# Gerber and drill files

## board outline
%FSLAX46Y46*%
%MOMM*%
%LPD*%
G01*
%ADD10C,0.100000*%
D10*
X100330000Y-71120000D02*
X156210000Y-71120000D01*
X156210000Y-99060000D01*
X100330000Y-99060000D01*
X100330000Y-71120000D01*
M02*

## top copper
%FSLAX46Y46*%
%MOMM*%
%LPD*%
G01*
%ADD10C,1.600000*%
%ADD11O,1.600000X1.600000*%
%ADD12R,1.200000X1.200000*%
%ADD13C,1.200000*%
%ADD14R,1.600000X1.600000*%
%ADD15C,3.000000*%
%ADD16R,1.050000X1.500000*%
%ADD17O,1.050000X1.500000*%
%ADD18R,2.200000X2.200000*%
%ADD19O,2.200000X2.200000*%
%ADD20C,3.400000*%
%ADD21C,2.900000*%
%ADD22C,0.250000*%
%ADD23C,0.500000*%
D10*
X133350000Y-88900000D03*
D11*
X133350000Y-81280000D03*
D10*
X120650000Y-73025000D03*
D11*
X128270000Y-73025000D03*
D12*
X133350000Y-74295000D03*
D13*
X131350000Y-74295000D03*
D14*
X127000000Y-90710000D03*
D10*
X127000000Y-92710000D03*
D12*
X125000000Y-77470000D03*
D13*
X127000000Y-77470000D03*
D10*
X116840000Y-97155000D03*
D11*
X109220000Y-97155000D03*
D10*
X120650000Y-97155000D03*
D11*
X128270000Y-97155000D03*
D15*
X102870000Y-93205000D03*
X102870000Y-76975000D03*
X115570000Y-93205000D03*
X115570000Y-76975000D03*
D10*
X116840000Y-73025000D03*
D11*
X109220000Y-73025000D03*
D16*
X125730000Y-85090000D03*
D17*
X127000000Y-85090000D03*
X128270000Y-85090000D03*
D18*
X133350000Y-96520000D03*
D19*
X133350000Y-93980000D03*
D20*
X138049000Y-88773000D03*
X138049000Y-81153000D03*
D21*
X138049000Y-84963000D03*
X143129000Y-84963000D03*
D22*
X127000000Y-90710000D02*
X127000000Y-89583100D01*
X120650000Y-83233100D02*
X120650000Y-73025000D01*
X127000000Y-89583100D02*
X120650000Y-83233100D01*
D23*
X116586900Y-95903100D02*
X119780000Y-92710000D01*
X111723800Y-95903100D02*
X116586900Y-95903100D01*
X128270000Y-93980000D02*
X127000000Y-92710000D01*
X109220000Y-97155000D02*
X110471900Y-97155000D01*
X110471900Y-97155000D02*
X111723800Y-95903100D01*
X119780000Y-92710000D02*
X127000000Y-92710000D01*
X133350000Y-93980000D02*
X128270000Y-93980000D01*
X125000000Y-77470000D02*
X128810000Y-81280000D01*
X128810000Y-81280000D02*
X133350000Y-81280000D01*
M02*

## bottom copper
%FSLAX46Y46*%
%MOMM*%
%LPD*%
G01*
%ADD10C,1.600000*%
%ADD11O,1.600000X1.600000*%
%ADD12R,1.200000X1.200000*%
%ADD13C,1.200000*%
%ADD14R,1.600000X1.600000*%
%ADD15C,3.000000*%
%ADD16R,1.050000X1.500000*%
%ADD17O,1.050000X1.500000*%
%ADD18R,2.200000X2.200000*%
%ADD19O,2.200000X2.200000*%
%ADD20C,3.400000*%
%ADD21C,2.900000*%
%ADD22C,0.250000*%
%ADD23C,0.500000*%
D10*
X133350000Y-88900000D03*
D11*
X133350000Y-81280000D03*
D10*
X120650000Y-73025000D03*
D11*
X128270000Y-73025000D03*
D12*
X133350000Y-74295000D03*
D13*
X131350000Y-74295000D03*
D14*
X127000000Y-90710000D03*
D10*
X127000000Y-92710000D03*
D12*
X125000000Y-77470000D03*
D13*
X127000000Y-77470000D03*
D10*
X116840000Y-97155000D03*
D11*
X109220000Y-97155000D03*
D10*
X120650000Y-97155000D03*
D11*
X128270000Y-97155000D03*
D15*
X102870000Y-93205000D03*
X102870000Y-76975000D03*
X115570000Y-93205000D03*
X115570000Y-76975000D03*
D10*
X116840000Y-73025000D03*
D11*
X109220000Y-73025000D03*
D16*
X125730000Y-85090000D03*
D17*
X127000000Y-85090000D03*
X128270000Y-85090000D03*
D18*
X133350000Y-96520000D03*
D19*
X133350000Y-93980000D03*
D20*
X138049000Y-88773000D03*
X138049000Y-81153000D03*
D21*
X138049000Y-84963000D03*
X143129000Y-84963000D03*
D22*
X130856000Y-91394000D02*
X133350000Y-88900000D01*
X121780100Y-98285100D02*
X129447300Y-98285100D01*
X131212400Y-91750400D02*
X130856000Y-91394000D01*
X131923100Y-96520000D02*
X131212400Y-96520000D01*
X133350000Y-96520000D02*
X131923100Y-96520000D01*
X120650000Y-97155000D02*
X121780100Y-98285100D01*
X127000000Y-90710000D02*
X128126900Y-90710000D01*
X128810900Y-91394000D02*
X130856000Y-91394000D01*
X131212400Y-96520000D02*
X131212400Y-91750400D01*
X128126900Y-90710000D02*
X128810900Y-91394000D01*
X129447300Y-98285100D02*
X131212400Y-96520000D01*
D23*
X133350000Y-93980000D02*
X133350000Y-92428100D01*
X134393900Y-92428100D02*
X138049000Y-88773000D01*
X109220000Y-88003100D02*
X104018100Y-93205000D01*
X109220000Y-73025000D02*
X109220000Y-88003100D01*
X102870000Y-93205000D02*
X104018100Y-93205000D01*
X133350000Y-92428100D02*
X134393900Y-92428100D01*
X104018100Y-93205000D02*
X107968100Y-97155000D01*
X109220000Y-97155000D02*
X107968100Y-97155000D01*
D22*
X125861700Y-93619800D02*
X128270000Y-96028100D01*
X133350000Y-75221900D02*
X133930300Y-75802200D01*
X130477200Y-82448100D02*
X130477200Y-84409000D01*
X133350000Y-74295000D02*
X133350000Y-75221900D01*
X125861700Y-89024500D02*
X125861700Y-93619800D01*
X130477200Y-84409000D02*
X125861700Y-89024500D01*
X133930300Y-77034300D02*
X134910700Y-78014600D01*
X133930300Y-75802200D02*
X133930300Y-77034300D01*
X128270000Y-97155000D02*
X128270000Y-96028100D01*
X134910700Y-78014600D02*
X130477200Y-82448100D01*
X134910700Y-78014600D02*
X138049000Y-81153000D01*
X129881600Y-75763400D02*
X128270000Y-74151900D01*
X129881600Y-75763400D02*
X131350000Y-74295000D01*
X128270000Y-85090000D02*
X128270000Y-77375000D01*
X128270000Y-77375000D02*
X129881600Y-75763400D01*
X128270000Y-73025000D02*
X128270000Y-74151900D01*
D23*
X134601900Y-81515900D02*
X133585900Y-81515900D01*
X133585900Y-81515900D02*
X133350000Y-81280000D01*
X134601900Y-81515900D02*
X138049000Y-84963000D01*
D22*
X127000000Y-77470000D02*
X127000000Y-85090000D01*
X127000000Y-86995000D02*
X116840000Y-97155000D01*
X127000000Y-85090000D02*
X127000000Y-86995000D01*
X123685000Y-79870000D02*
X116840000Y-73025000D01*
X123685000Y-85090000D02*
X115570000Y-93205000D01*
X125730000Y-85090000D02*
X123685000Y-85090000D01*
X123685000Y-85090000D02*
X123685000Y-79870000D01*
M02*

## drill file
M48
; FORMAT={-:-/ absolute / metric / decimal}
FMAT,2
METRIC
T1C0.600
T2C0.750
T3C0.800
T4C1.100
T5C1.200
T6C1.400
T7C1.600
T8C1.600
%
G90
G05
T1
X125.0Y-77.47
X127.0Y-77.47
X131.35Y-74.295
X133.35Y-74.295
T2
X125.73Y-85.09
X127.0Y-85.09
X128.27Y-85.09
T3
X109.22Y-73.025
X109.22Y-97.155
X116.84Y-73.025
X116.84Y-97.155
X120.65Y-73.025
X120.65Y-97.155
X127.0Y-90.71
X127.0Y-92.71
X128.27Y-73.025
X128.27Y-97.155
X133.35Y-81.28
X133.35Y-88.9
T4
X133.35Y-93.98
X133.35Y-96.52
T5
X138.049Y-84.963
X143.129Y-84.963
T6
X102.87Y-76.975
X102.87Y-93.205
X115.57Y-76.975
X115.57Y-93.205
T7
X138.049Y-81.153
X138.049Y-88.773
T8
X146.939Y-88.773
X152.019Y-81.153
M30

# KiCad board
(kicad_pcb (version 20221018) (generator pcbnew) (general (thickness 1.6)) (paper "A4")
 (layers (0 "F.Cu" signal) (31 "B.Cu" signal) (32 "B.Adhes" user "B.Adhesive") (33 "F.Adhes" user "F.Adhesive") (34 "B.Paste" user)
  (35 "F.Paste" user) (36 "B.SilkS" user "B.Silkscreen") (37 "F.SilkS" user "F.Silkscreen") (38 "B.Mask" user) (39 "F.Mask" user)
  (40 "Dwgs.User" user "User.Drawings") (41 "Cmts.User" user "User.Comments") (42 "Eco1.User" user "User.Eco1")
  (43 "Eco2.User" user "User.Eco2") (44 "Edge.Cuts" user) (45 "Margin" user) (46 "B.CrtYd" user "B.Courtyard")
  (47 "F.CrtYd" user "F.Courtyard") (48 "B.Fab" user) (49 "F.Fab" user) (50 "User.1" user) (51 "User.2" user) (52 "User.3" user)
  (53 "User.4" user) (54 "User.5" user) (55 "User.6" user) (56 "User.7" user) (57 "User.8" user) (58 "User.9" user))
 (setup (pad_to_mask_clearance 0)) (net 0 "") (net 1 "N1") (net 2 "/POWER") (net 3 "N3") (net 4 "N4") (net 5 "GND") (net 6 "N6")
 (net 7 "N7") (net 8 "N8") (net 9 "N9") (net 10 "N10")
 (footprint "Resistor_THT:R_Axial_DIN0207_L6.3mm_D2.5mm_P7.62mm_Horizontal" (layer "F.Cu") (at 133.35 88.9 90)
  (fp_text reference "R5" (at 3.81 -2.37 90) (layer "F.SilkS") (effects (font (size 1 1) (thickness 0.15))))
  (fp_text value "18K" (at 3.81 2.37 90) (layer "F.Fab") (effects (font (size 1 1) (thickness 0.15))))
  (pad "1" thru_hole circle (at 0 0 90) (size 1.6 1.6) (drill 0.8) (layers "*.Cu" "*.Mask") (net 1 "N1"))
  (pad "2" thru_hole oval (at 7.62 0 90) (size 1.6 1.6) (drill 0.8) (layers "*.Cu" "*.Mask") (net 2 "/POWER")))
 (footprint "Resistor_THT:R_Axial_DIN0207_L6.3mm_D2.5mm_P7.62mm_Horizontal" (layer "F.Cu") (at 120.65 73.025)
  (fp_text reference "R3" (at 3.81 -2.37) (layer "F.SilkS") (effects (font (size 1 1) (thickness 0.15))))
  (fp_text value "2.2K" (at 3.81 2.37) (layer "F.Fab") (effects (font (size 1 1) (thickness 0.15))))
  (pad "1" thru_hole circle (at 0 0) (size 1.6 1.6) (drill 0.8) (layers "*.Cu" "*.Mask") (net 1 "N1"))
  (pad "2" thru_hole oval (at 7.62 0) (size 1.6 1.6) (drill 0.8) (layers "*.Cu" "*.Mask") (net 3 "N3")))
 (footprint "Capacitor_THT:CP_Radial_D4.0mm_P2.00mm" (layer "F.Cu") (at 133.35 74.295 180)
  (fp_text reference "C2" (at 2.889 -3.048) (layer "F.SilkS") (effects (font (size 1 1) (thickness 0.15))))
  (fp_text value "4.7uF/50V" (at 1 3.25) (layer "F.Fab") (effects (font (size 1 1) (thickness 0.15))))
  (pad "1" thru_hole rect (at 0 0 180) (size 1.2 1.2) (drill 0.6) (layers "*.Cu" "*.Mask") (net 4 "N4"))
  (pad "2" thru_hole circle (at 2 0 180) (size 1.2 1.2) (drill 0.6) (layers "*.Cu" "*.Mask") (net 3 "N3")))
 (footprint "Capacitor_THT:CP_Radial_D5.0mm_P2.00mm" (layer "F.Cu") (at 127 90.71 -90)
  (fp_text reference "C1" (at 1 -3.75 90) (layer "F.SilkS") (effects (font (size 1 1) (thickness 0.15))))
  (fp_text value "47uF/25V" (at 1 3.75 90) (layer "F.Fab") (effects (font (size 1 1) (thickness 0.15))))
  (pad "1" thru_hole rect (at 0 0 270) (size 1.6 1.6) (drill 0.8) (layers "*.Cu" "*.Mask") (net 1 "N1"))
  (pad "2" thru_hole circle (at 2 0 270) (size 1.6 1.6) (drill 0.8) (layers "*.Cu" "*.Mask") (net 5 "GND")))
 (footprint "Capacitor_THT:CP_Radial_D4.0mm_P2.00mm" (layer "F.Cu") (at 125 77.47)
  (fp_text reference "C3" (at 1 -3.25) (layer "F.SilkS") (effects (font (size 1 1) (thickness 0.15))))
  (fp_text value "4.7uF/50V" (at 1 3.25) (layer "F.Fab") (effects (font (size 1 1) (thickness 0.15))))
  (pad "1" thru_hole rect (at 0 0) (size 1.2 1.2) (drill 0.6) (layers "*.Cu" "*.Mask") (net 2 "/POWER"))
  (pad "2" thru_hole circle (at 2 0) (size 1.2 1.2) (drill 0.6) (layers "*.Cu" "*.Mask") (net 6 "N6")))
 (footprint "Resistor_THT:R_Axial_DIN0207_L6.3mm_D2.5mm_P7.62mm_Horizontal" (layer "F.Cu") (at 116.84 97.155 180)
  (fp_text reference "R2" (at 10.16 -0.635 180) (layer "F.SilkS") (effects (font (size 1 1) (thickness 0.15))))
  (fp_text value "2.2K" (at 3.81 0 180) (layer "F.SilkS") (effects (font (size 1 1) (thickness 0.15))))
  (pad "1" thru_hole circle (at 0 0 180) (size 1.6 1.6) (drill 0.8) (layers "*.Cu" "*.Mask") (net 6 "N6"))
  (pad "2" thru_hole oval (at 7.62 0 180) (size 1.6 1.6) (drill 0.8) (layers "*.Cu" "*.Mask") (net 5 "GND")))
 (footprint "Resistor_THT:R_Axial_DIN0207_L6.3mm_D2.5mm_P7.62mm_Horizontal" (layer "F.Cu") (at 120.65 97.155)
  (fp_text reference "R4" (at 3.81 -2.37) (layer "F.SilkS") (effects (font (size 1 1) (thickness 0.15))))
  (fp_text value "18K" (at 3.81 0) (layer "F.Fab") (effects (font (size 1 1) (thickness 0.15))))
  (pad "1" thru_hole circle (at 0 0) (size 1.6 1.6) (drill 0.8) (layers "*.Cu" "*.Mask") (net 1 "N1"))
  (pad "2" thru_hole oval (at 7.62 0) (size 1.6 1.6) (drill 0.8) (layers "*.Cu" "*.Mask") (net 4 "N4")))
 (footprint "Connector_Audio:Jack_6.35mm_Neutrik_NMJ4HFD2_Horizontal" (layer "F.Cu") (at 115.57 93.205 180)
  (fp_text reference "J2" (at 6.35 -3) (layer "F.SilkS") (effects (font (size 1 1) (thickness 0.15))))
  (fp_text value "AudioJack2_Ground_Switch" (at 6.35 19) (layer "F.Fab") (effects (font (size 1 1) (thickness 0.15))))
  (pad "S" thru_hole circle (at 12.7 0 180) (size 3 3) (drill 1.4) (layers "*.Cu" "*.Mask") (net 5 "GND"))
  (pad "SN" thru_hole circle (at 12.7 16.23 180) (size 3 3) (drill 1.4) (layers "*.Cu" "*.Mask") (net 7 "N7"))
  (pad "T" thru_hole circle (at 0 0 180) (size 3 3) (drill 1.4) (layers "*.Cu" "*.Mask") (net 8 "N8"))
  (pad "TN" thru_hole circle (at 0 16.23 180) (size 3 3) (drill 1.4) (layers "*.Cu" "*.Mask") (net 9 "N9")))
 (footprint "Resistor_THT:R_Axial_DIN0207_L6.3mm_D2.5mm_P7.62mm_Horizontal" (layer "F.Cu") (at 116.84 73.025 180)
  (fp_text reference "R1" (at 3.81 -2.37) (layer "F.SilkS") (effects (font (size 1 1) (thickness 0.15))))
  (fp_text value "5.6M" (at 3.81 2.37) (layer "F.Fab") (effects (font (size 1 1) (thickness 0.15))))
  (pad "1" thru_hole circle (at 0 0 180) (size 1.6 1.6) (drill 0.8) (layers "*.Cu" "*.Mask") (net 8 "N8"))
  (pad "2" thru_hole oval (at 7.62 0 180) (size 1.6 1.6) (drill 0.8) (layers "*.Cu" "*.Mask") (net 5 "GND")))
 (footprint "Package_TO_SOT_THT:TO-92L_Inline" (layer "F.Cu") (at 125.73 85.09)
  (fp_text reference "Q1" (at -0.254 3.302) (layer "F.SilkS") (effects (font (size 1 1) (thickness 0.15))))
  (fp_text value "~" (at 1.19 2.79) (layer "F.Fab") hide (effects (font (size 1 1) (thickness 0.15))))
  (pad "1" thru_hole rect (at 0 0) (size 1.05 1.5) (drill 0.75) (layers "*.Cu" "*.Mask") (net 8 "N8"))
  (pad "2" thru_hole oval (at 1.27 0) (size 1.05 1.5) (drill 0.75) (layers "*.Cu" "*.Mask") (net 6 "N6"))
  (pad "3" thru_hole oval (at 2.54 0) (size 1.05 1.5) (drill 0.75) (layers "*.Cu" "*.Mask") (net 3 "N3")))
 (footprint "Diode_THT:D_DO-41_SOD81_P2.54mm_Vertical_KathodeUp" (layer "F.Cu") (at 133.35 96.52 90)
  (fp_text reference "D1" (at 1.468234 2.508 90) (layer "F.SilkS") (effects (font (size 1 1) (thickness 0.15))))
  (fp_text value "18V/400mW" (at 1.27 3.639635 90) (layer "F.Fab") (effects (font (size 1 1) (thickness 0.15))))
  (pad "1" thru_hole rect (at 0 0 90) (size 2.2 2.2) (drill 1.1) (layers "*.Cu" "*.Mask") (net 1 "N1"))
  (pad "2" thru_hole oval (at 2.54 0 90) (size 2.2 2.2) (drill 1.1) (layers "*.Cu" "*.Mask") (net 5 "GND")))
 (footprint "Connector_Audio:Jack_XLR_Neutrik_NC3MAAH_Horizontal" (layer "F.Cu") (at 138.049 88.773 90)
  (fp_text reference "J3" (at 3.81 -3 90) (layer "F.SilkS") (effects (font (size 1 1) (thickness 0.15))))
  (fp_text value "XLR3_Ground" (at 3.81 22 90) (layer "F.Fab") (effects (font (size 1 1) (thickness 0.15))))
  (pad "" np_thru_hole circle (at 0 8.89 90) (size 1.6 1.6) (drill 1.6) (layers "*.Cu" "*.Mask"))
  (pad "" np_thru_hole circle (at 7.62 13.97 90) (size 1.6 1.6) (drill 1.6) (layers "*.Cu" "*.Mask"))
  (pad "1" thru_hole circle (at 0 0 90) (size 3.4 3.4) (drill 1.6) (layers "*.Cu" "*.Mask") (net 5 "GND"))
  (pad "2" thru_hole circle (at 7.62 0 90) (size 3.4 3.4) (drill 1.6) (layers "*.Cu" "*.Mask") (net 4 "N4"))
  (pad "3" thru_hole circle (at 3.81 0 90) (size 2.9 2.9) (drill 1.2) (layers "*.Cu" "*.Mask") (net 2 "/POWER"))
  (pad "G" thru_hole circle (at 3.81 5.08 90) (size 2.9 2.9) (drill 1.2) (layers "*.Cu" "*.Mask") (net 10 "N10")))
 (gr_rect (start 100.33 71.12) (end 156.21 99.06) (stroke (width 0.1) (type default)) (fill none) (layer "Edge.Cuts"))
 (segment (start 127 90.71) (end 127 89.5831) (width 0.25) (layer "F.Cu") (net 1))
 (segment (start 120.65 83.2331) (end 120.65 73.025) (width 0.25) (layer "F.Cu") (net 1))
 (segment (start 127 89.5831) (end 120.65 83.2331) (width 0.25) (layer "F.Cu") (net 1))
 (segment (start 130.856 91.394) (end 133.35 88.9) (width 0.25) (layer "B.Cu") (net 1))
 (segment (start 121.7801 98.2851) (end 129.4473 98.2851) (width 0.25) (layer "B.Cu") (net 1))
 (segment (start 131.2124 91.7504) (end 130.856 91.394) (width 0.25) (layer "B.Cu") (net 1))
 (segment (start 131.9231 96.52) (end 131.2124 96.52) (width 0.25) (layer "B.Cu") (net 1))
 (segment (start 133.35 96.52) (end 131.9231 96.52) (width 0.25) (layer "B.Cu") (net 1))
 (segment (start 120.65 97.155) (end 121.7801 98.2851) (width 0.25) (layer "B.Cu") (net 1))
 (segment (start 127 90.71) (end 128.1269 90.71) (width 0.25) (layer "B.Cu") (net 1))
 (segment (start 128.8109 91.394) (end 130.856 91.394) (width 0.25) (layer "B.Cu") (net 1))
 (segment (start 131.2124 96.52) (end 131.2124 91.7504) (width 0.25) (layer "B.Cu") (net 1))
 (segment (start 128.1269 90.71) (end 128.8109 91.394) (width 0.25) (layer "B.Cu") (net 1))
 (segment (start 129.4473 98.2851) (end 131.2124 96.52) (width 0.25) (layer "B.Cu") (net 1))
 (segment (start 116.5869 95.9031) (end 119.78 92.71) (width 0.5) (layer "F.Cu") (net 5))
 (segment (start 111.7238 95.9031) (end 116.5869 95.9031) (width 0.5) (layer "F.Cu") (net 5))
 (segment (start 128.27 93.98) (end 127 92.71) (width 0.5) (layer "F.Cu") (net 5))
 (segment (start 109.22 97.155) (end 110.4719 97.155) (width 0.5) (layer "F.Cu") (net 5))
 (segment (start 110.4719 97.155) (end 111.7238 95.9031) (width 0.5) (layer "F.Cu") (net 5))
 (segment (start 119.78 92.71) (end 127 92.71) (width 0.5) (layer "F.Cu") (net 5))
 (segment (start 133.35 93.98) (end 128.27 93.98) (width 0.5) (layer "F.Cu") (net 5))
 (segment (start 133.35 93.98) (end 133.35 92.4281) (width 0.5) (layer "B.Cu") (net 5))
 (segment (start 134.3939 92.4281) (end 138.049 88.773) (width 0.5) (layer "B.Cu") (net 5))
 (segment (start 109.22 88.0031) (end 104.0181 93.205) (width 0.5) (layer "B.Cu") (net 5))
 (segment (start 109.22 73.025) (end 109.22 88.0031) (width 0.5) (layer "B.Cu") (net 5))
 (segment (start 102.87 93.205) (end 104.0181 93.205) (width 0.5) (layer "B.Cu") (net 5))
 (segment (start 133.35 92.4281) (end 134.3939 92.4281) (width 0.5) (layer "B.Cu") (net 5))
 (segment (start 104.0181 93.205) (end 107.9681 97.155) (width 0.5) (layer "B.Cu") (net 5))
 (segment (start 109.22 97.155) (end 107.9681 97.155) (width 0.5) (layer "B.Cu") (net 5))
 (segment (start 125.8617 93.6198) (end 128.27 96.0281) (width 0.25) (layer "B.Cu") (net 4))
 (segment (start 133.35 75.2219) (end 133.9303 75.8022) (width 0.25) (layer "B.Cu") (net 4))
 (segment (start 130.4772 82.4481) (end 130.4772 84.409) (width 0.25) (layer "B.Cu") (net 4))
 (segment (start 133.35 74.295) (end 133.35 75.2219) (width 0.25) (layer "B.Cu") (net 4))
 (segment (start 125.8617 89.0245) (end 125.8617 93.6198) (width 0.25) (layer "B.Cu") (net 4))
 (segment (start 130.4772 84.409) (end 125.8617 89.0245) (width 0.25) (layer "B.Cu") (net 4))
 (segment (start 133.9303 77.0343) (end 134.9107 78.0146) (width 0.25) (layer "B.Cu") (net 4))
 (segment (start 133.9303 75.8022) (end 133.9303 77.0343) (width 0.25) (layer "B.Cu") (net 4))
 (segment (start 128.27 97.155) (end 128.27 96.0281) (width 0.25) (layer "B.Cu") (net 4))
 (segment (start 134.9107 78.0146) (end 130.4772 82.4481) (width 0.25) (layer "B.Cu") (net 4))
 (segment (start 134.9107 78.0146) (end 138.049 81.153) (width 0.25) (layer "B.Cu") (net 4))
 (segment (start 129.8816 75.7634) (end 128.27 74.1519) (width 0.25) (layer "B.Cu") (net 3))
 (segment (start 129.8816 75.7634) (end 131.35 74.295) (width 0.25) (layer "B.Cu") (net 3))
 (segment (start 128.27 85.09) (end 128.27 77.375) (width 0.25) (layer "B.Cu") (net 3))
 (segment (start 128.27 77.375) (end 129.8816 75.7634) (width 0.25) (layer "B.Cu") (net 3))
 (segment (start 128.27 73.025) (end 128.27 74.1519) (width 0.25) (layer "B.Cu") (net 3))
 (segment (start 125 77.47) (end 128.81 81.28) (width 0.5) (layer "F.Cu") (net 2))
 (segment (start 128.81 81.28) (end 133.35 81.28) (width 0.5) (layer "F.Cu") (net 2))
 (segment (start 134.6019 81.5159) (end 133.5859 81.5159) (width 0.5) (layer "B.Cu") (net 2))
 (segment (start 133.5859 81.5159) (end 133.35 81.28) (width 0.5) (layer "B.Cu") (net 2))
 (segment (start 134.6019 81.5159) (end 138.049 84.963) (width 0.5) (layer "B.Cu") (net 2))
 (segment (start 127 77.47) (end 127 85.09) (width 0.25) (layer "B.Cu") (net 6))
 (segment (start 127 86.995) (end 116.84 97.155) (width 0.25) (layer "B.Cu") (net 6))
 (segment (start 127 85.09) (end 127 86.995) (width 0.25) (layer "B.Cu") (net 6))
 (segment (start 123.685 79.87) (end 116.84 73.025) (width 0.25) (layer "B.Cu") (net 8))
 (segment (start 123.685 85.09) (end 115.57 93.205) (width 0.25) (layer "B.Cu") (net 8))
 (segment (start 125.73 85.09) (end 123.685 85.09) (width 0.25) (layer "B.Cu") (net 8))
 (segment (start 123.685 85.09) (end 123.685 79.87) (width 0.25) (layer "B.Cu") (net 8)))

